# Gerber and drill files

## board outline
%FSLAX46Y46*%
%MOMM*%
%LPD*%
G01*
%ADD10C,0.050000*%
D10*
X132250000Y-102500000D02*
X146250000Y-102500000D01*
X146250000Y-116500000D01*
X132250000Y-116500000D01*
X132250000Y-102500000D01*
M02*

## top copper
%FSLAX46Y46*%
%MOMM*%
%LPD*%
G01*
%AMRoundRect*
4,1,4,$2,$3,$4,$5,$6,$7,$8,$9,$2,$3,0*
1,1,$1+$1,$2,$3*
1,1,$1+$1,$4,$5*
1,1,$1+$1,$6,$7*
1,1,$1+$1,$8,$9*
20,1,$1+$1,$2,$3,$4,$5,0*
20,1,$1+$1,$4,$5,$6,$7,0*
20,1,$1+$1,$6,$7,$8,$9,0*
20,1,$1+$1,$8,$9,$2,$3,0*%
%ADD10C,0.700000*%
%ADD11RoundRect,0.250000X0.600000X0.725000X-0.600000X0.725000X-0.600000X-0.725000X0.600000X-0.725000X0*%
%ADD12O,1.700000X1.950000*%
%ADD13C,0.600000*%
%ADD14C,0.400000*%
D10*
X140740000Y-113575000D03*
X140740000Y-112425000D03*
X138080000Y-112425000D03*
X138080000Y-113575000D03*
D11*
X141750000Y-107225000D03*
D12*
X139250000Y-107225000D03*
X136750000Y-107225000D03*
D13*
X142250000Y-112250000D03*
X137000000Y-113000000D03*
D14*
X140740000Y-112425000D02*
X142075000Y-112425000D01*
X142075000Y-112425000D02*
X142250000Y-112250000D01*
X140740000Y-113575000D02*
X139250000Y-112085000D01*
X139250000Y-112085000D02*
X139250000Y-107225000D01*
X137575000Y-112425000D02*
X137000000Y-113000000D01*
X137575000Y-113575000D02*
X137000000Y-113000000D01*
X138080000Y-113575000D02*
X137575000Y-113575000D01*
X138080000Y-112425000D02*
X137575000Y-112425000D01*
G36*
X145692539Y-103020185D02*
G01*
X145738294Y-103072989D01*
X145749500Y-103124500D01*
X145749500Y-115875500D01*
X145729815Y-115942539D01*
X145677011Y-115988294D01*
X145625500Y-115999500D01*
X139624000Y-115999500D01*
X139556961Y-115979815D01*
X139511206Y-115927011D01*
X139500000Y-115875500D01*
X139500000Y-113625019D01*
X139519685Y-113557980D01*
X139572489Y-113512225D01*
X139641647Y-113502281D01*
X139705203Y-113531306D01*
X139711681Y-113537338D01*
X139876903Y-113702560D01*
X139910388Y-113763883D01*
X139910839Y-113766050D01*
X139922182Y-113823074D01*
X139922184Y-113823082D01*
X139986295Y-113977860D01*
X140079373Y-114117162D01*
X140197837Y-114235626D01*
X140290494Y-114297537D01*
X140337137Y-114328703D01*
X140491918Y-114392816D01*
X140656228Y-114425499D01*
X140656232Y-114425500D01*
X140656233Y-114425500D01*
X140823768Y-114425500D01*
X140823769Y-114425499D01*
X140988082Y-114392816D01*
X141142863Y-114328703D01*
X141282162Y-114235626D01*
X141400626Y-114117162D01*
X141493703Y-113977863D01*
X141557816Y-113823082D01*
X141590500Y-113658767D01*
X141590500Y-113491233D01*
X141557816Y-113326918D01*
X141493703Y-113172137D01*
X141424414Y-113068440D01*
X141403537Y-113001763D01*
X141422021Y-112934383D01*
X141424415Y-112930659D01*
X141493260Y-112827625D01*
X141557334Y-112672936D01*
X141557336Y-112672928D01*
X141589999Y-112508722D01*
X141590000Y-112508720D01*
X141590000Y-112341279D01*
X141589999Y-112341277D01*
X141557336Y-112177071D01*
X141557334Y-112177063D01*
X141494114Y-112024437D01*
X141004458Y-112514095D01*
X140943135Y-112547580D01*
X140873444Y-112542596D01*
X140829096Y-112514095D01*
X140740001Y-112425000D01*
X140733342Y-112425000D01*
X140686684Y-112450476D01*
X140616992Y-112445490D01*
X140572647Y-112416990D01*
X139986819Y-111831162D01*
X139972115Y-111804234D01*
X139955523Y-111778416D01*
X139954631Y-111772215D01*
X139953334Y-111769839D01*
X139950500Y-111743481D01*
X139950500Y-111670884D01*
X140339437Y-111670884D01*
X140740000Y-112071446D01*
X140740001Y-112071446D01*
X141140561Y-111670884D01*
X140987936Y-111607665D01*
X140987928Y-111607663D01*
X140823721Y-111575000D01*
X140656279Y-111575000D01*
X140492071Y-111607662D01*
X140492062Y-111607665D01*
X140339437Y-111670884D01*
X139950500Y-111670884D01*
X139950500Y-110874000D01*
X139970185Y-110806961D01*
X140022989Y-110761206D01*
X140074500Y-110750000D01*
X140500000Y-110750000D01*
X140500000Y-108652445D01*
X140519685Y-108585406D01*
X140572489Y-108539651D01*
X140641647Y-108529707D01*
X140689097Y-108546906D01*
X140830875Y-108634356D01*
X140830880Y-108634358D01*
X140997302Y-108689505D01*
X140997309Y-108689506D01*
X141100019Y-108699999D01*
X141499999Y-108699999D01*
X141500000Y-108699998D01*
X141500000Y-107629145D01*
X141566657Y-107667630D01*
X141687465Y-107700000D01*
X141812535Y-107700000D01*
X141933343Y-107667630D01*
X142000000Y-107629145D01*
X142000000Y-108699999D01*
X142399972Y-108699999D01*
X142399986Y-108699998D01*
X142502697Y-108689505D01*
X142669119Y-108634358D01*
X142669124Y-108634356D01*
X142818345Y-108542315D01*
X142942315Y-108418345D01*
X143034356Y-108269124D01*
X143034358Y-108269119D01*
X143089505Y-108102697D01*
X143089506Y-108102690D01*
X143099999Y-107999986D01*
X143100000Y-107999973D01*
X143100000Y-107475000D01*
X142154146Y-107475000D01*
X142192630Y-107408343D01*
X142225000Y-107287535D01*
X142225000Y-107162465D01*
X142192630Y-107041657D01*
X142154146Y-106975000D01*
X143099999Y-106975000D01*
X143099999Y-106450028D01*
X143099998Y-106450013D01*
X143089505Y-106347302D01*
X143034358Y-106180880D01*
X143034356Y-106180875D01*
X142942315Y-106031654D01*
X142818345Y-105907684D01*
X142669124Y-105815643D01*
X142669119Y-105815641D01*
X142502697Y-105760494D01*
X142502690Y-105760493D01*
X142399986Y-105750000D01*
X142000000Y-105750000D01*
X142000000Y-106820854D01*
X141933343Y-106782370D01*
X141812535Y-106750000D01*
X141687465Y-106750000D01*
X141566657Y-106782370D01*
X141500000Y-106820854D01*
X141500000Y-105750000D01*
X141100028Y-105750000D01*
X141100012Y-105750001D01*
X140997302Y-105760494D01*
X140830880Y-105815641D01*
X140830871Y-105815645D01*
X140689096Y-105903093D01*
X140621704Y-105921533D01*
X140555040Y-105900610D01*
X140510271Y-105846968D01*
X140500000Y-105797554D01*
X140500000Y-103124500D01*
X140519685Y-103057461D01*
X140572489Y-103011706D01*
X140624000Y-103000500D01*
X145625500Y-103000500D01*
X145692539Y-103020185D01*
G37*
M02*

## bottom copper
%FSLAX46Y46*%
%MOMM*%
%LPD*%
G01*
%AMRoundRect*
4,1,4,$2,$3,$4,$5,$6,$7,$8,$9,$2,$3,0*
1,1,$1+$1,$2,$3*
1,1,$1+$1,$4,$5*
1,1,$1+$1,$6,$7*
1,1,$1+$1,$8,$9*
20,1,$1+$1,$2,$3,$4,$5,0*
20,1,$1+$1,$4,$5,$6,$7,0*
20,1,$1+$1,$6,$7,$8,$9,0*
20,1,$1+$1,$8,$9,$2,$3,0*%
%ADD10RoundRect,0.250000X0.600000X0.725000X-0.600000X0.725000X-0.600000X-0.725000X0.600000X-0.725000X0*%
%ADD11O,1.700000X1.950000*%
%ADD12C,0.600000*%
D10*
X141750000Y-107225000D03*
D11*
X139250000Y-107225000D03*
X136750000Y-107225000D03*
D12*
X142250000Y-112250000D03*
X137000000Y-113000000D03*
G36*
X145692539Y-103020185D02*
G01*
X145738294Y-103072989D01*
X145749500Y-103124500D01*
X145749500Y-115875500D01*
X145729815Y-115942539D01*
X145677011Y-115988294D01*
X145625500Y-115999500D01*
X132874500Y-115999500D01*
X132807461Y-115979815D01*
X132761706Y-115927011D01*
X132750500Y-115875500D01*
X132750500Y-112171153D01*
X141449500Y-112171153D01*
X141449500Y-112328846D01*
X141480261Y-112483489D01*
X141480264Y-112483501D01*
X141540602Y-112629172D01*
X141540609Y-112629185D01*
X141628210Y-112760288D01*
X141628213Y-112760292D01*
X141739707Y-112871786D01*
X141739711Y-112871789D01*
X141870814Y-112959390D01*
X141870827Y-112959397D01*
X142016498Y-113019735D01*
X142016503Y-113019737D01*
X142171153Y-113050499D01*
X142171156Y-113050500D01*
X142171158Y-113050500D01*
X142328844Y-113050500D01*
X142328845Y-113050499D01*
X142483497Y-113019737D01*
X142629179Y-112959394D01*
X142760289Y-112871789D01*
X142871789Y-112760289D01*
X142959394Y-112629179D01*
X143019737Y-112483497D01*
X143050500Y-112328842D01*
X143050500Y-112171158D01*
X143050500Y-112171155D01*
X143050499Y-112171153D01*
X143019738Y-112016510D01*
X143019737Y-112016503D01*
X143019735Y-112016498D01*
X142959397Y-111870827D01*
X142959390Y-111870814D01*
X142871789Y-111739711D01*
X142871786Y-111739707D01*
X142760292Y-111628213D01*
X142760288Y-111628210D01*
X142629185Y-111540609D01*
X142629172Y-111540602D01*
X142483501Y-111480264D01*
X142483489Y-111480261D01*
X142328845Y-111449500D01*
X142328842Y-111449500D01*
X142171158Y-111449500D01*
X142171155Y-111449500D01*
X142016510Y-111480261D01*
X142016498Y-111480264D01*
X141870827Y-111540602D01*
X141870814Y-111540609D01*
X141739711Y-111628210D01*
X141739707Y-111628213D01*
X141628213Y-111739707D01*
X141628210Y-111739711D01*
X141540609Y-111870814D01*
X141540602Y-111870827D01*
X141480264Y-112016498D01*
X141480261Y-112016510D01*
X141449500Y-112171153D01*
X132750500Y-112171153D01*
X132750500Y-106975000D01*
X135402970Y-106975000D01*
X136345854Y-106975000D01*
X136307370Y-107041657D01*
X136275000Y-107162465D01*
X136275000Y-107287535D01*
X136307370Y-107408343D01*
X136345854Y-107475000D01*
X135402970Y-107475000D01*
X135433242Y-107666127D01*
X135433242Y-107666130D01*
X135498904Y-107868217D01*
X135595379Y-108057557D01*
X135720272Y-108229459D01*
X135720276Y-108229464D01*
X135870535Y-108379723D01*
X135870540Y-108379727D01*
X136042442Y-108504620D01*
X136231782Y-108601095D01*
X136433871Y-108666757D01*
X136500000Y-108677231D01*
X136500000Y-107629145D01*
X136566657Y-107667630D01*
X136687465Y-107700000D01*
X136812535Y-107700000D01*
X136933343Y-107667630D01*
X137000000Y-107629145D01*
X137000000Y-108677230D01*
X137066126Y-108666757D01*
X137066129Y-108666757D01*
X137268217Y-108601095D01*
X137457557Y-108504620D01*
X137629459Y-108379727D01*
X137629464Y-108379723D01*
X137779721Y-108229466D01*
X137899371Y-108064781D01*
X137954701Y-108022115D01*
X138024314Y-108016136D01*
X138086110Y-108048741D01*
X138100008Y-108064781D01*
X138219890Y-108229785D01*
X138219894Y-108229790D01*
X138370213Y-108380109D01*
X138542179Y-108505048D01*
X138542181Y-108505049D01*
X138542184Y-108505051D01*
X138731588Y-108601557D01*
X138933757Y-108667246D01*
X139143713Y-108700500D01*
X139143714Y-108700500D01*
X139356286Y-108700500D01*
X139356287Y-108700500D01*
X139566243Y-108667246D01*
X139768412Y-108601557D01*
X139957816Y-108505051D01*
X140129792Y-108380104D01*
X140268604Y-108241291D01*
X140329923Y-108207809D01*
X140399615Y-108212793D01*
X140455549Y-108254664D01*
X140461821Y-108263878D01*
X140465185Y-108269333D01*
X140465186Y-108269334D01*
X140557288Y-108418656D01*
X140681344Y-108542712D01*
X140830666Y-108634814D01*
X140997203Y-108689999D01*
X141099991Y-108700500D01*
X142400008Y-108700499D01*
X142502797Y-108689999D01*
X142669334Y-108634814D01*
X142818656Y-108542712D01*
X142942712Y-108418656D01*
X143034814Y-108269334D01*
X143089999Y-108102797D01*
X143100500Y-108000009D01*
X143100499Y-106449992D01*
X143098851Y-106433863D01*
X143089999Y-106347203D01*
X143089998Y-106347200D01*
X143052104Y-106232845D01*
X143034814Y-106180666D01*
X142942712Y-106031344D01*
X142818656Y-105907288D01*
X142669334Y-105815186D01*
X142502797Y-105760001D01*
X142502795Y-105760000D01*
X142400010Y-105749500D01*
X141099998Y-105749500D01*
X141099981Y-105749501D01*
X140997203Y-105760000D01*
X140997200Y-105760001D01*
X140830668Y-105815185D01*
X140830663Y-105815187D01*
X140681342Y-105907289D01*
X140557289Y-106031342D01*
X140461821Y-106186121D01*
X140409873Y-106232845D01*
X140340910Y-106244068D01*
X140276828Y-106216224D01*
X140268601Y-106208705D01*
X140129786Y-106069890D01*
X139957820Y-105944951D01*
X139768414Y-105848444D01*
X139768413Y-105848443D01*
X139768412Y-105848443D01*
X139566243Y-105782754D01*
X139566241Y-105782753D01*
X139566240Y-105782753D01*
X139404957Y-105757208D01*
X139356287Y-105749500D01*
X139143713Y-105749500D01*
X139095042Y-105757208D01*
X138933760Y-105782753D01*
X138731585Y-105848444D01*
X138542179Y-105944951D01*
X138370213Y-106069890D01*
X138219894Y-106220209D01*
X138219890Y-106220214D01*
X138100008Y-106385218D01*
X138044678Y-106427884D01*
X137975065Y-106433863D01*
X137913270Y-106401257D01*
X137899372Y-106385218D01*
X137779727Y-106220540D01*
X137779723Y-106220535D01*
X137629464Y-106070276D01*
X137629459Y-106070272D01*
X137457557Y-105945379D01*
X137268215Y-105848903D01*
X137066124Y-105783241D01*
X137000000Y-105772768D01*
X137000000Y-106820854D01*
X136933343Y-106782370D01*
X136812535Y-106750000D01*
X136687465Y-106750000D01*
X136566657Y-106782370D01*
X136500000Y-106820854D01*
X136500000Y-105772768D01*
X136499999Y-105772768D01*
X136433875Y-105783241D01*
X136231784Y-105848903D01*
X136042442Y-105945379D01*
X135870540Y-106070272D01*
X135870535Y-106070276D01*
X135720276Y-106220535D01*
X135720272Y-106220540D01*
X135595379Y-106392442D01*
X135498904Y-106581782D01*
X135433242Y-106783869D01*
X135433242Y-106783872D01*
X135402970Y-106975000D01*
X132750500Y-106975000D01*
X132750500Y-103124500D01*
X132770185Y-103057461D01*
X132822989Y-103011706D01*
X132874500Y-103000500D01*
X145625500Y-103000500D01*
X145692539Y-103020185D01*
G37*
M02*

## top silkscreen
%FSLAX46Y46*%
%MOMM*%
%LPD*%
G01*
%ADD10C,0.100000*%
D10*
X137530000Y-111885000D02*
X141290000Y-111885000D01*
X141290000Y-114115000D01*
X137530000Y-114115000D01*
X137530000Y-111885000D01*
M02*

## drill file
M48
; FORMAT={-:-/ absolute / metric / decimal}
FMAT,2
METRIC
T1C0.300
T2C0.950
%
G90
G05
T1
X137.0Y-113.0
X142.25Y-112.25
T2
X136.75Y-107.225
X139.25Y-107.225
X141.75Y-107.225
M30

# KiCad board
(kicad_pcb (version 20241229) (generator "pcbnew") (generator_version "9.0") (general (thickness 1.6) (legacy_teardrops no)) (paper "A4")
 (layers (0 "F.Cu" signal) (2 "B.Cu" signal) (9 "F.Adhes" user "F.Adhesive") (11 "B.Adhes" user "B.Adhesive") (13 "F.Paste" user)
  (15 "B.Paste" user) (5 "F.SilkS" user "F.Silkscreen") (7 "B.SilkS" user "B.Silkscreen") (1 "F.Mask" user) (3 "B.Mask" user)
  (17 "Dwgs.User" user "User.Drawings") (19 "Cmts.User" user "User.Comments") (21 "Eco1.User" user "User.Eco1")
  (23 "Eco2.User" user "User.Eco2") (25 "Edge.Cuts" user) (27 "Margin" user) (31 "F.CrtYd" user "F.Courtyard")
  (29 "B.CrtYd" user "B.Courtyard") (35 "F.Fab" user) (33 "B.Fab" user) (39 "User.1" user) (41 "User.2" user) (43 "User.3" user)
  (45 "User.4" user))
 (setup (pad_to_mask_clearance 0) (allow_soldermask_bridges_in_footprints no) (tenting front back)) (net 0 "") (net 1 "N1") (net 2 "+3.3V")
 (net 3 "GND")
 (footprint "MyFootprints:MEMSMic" (layer "F.Cu") (at 136.91 113.115 -90)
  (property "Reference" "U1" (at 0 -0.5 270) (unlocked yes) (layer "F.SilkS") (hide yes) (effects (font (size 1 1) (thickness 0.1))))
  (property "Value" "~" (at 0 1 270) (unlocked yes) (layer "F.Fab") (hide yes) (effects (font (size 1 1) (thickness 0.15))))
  (fp_rect (start -1.23 -4.38) (end 1 -0.62) (stroke (width 0.1) (type solid)) (fill no) (layer "F.SilkS"))
  (pad "1" smd circle (at 0.46 -3.83 270) (size 0.7 0.7) (layers "F.Cu" "F.Mask" "F.Paste") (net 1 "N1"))
  (pad "2" smd circle (at -0.69 -3.83 270) (size 0.7 0.7) (layers "F.Cu" "F.Mask" "F.Paste") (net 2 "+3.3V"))
  (pad "3" smd circle (at -0.69 -1.17 270) (size 0.7 0.7) (layers "F.Cu" "F.Mask" "F.Paste") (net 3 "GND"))
  (pad "4" smd circle (at 0.46 -1.17 270) (size 0.7 0.7) (layers "F.Cu" "F.Mask" "F.Paste") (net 3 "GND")))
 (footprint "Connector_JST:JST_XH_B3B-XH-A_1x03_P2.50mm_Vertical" (layer "B.Cu") (at 141.75 107.225 180)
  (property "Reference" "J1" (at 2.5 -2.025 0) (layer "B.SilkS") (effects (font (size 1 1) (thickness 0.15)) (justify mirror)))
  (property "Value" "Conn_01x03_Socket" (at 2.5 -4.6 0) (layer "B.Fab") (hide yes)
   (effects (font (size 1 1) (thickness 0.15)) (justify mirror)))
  (pad "1" thru_hole roundrect (at 0 0 180) (size 1.7 1.95) (drill 0.95) (layers "*.Cu" "*.Mask") (remove_unused_layers no)
   (roundrect_rratio 0.147059) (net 2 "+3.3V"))
  (pad "2" thru_hole oval (at 2.5 0 180) (size 1.7 1.95) (drill 0.95) (layers "*.Cu" "*.Mask") (remove_unused_layers no) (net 1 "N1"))
  (pad "3" thru_hole oval (at 5 0 180) (size 1.7 1.95) (drill 0.95) (layers "*.Cu" "*.Mask") (remove_unused_layers no) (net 3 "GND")))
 (gr_rect (start 132.25 102.5) (end 146.25 116.5) (stroke (width 0.05) (type default)) (fill no) (layer "Edge.Cuts"))
 (segment (start 140.74 112.425) (end 142.075 112.425) (width 0.4) (layer "F.Cu") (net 2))
 (segment (start 142.075 112.425) (end 142.25 112.25) (width 0.4) (layer "F.Cu") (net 2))
 (via (at 142.25 112.25) (size 0.6) (drill 0.3) (layers "F.Cu" "B.Cu") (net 2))
 (segment (start 140.74 113.575) (end 139.25 112.085) (width 0.4) (layer "F.Cu") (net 1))
 (segment (start 139.25 112.085) (end 139.25 107.225) (width 0.4) (layer "F.Cu") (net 1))
 (segment (start 137.575 112.425) (end 137 113) (width 0.4) (layer "F.Cu") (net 3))
 (segment (start 137.575 113.575) (end 137 113) (width 0.4) (layer "F.Cu") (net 3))
 (segment (start 138.08 113.575) (end 137.575 113.575) (width 0.4) (layer "F.Cu") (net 3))
 (segment (start 138.08 112.425) (end 137.575 112.425) (width 0.4) (layer "F.Cu") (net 3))
 (via (at 137 113) (size 0.6) (drill 0.3) (layers "F.Cu" "B.Cu") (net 3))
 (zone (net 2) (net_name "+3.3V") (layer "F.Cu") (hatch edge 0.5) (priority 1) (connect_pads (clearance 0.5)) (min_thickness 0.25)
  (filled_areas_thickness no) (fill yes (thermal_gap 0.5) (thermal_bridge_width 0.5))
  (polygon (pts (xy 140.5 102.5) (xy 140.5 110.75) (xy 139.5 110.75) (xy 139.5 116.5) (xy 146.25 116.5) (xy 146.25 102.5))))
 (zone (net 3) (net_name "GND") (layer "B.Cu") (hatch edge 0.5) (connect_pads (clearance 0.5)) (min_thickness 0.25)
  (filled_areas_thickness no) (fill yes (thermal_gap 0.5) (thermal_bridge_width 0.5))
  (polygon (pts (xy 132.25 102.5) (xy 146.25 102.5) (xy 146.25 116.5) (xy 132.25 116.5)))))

